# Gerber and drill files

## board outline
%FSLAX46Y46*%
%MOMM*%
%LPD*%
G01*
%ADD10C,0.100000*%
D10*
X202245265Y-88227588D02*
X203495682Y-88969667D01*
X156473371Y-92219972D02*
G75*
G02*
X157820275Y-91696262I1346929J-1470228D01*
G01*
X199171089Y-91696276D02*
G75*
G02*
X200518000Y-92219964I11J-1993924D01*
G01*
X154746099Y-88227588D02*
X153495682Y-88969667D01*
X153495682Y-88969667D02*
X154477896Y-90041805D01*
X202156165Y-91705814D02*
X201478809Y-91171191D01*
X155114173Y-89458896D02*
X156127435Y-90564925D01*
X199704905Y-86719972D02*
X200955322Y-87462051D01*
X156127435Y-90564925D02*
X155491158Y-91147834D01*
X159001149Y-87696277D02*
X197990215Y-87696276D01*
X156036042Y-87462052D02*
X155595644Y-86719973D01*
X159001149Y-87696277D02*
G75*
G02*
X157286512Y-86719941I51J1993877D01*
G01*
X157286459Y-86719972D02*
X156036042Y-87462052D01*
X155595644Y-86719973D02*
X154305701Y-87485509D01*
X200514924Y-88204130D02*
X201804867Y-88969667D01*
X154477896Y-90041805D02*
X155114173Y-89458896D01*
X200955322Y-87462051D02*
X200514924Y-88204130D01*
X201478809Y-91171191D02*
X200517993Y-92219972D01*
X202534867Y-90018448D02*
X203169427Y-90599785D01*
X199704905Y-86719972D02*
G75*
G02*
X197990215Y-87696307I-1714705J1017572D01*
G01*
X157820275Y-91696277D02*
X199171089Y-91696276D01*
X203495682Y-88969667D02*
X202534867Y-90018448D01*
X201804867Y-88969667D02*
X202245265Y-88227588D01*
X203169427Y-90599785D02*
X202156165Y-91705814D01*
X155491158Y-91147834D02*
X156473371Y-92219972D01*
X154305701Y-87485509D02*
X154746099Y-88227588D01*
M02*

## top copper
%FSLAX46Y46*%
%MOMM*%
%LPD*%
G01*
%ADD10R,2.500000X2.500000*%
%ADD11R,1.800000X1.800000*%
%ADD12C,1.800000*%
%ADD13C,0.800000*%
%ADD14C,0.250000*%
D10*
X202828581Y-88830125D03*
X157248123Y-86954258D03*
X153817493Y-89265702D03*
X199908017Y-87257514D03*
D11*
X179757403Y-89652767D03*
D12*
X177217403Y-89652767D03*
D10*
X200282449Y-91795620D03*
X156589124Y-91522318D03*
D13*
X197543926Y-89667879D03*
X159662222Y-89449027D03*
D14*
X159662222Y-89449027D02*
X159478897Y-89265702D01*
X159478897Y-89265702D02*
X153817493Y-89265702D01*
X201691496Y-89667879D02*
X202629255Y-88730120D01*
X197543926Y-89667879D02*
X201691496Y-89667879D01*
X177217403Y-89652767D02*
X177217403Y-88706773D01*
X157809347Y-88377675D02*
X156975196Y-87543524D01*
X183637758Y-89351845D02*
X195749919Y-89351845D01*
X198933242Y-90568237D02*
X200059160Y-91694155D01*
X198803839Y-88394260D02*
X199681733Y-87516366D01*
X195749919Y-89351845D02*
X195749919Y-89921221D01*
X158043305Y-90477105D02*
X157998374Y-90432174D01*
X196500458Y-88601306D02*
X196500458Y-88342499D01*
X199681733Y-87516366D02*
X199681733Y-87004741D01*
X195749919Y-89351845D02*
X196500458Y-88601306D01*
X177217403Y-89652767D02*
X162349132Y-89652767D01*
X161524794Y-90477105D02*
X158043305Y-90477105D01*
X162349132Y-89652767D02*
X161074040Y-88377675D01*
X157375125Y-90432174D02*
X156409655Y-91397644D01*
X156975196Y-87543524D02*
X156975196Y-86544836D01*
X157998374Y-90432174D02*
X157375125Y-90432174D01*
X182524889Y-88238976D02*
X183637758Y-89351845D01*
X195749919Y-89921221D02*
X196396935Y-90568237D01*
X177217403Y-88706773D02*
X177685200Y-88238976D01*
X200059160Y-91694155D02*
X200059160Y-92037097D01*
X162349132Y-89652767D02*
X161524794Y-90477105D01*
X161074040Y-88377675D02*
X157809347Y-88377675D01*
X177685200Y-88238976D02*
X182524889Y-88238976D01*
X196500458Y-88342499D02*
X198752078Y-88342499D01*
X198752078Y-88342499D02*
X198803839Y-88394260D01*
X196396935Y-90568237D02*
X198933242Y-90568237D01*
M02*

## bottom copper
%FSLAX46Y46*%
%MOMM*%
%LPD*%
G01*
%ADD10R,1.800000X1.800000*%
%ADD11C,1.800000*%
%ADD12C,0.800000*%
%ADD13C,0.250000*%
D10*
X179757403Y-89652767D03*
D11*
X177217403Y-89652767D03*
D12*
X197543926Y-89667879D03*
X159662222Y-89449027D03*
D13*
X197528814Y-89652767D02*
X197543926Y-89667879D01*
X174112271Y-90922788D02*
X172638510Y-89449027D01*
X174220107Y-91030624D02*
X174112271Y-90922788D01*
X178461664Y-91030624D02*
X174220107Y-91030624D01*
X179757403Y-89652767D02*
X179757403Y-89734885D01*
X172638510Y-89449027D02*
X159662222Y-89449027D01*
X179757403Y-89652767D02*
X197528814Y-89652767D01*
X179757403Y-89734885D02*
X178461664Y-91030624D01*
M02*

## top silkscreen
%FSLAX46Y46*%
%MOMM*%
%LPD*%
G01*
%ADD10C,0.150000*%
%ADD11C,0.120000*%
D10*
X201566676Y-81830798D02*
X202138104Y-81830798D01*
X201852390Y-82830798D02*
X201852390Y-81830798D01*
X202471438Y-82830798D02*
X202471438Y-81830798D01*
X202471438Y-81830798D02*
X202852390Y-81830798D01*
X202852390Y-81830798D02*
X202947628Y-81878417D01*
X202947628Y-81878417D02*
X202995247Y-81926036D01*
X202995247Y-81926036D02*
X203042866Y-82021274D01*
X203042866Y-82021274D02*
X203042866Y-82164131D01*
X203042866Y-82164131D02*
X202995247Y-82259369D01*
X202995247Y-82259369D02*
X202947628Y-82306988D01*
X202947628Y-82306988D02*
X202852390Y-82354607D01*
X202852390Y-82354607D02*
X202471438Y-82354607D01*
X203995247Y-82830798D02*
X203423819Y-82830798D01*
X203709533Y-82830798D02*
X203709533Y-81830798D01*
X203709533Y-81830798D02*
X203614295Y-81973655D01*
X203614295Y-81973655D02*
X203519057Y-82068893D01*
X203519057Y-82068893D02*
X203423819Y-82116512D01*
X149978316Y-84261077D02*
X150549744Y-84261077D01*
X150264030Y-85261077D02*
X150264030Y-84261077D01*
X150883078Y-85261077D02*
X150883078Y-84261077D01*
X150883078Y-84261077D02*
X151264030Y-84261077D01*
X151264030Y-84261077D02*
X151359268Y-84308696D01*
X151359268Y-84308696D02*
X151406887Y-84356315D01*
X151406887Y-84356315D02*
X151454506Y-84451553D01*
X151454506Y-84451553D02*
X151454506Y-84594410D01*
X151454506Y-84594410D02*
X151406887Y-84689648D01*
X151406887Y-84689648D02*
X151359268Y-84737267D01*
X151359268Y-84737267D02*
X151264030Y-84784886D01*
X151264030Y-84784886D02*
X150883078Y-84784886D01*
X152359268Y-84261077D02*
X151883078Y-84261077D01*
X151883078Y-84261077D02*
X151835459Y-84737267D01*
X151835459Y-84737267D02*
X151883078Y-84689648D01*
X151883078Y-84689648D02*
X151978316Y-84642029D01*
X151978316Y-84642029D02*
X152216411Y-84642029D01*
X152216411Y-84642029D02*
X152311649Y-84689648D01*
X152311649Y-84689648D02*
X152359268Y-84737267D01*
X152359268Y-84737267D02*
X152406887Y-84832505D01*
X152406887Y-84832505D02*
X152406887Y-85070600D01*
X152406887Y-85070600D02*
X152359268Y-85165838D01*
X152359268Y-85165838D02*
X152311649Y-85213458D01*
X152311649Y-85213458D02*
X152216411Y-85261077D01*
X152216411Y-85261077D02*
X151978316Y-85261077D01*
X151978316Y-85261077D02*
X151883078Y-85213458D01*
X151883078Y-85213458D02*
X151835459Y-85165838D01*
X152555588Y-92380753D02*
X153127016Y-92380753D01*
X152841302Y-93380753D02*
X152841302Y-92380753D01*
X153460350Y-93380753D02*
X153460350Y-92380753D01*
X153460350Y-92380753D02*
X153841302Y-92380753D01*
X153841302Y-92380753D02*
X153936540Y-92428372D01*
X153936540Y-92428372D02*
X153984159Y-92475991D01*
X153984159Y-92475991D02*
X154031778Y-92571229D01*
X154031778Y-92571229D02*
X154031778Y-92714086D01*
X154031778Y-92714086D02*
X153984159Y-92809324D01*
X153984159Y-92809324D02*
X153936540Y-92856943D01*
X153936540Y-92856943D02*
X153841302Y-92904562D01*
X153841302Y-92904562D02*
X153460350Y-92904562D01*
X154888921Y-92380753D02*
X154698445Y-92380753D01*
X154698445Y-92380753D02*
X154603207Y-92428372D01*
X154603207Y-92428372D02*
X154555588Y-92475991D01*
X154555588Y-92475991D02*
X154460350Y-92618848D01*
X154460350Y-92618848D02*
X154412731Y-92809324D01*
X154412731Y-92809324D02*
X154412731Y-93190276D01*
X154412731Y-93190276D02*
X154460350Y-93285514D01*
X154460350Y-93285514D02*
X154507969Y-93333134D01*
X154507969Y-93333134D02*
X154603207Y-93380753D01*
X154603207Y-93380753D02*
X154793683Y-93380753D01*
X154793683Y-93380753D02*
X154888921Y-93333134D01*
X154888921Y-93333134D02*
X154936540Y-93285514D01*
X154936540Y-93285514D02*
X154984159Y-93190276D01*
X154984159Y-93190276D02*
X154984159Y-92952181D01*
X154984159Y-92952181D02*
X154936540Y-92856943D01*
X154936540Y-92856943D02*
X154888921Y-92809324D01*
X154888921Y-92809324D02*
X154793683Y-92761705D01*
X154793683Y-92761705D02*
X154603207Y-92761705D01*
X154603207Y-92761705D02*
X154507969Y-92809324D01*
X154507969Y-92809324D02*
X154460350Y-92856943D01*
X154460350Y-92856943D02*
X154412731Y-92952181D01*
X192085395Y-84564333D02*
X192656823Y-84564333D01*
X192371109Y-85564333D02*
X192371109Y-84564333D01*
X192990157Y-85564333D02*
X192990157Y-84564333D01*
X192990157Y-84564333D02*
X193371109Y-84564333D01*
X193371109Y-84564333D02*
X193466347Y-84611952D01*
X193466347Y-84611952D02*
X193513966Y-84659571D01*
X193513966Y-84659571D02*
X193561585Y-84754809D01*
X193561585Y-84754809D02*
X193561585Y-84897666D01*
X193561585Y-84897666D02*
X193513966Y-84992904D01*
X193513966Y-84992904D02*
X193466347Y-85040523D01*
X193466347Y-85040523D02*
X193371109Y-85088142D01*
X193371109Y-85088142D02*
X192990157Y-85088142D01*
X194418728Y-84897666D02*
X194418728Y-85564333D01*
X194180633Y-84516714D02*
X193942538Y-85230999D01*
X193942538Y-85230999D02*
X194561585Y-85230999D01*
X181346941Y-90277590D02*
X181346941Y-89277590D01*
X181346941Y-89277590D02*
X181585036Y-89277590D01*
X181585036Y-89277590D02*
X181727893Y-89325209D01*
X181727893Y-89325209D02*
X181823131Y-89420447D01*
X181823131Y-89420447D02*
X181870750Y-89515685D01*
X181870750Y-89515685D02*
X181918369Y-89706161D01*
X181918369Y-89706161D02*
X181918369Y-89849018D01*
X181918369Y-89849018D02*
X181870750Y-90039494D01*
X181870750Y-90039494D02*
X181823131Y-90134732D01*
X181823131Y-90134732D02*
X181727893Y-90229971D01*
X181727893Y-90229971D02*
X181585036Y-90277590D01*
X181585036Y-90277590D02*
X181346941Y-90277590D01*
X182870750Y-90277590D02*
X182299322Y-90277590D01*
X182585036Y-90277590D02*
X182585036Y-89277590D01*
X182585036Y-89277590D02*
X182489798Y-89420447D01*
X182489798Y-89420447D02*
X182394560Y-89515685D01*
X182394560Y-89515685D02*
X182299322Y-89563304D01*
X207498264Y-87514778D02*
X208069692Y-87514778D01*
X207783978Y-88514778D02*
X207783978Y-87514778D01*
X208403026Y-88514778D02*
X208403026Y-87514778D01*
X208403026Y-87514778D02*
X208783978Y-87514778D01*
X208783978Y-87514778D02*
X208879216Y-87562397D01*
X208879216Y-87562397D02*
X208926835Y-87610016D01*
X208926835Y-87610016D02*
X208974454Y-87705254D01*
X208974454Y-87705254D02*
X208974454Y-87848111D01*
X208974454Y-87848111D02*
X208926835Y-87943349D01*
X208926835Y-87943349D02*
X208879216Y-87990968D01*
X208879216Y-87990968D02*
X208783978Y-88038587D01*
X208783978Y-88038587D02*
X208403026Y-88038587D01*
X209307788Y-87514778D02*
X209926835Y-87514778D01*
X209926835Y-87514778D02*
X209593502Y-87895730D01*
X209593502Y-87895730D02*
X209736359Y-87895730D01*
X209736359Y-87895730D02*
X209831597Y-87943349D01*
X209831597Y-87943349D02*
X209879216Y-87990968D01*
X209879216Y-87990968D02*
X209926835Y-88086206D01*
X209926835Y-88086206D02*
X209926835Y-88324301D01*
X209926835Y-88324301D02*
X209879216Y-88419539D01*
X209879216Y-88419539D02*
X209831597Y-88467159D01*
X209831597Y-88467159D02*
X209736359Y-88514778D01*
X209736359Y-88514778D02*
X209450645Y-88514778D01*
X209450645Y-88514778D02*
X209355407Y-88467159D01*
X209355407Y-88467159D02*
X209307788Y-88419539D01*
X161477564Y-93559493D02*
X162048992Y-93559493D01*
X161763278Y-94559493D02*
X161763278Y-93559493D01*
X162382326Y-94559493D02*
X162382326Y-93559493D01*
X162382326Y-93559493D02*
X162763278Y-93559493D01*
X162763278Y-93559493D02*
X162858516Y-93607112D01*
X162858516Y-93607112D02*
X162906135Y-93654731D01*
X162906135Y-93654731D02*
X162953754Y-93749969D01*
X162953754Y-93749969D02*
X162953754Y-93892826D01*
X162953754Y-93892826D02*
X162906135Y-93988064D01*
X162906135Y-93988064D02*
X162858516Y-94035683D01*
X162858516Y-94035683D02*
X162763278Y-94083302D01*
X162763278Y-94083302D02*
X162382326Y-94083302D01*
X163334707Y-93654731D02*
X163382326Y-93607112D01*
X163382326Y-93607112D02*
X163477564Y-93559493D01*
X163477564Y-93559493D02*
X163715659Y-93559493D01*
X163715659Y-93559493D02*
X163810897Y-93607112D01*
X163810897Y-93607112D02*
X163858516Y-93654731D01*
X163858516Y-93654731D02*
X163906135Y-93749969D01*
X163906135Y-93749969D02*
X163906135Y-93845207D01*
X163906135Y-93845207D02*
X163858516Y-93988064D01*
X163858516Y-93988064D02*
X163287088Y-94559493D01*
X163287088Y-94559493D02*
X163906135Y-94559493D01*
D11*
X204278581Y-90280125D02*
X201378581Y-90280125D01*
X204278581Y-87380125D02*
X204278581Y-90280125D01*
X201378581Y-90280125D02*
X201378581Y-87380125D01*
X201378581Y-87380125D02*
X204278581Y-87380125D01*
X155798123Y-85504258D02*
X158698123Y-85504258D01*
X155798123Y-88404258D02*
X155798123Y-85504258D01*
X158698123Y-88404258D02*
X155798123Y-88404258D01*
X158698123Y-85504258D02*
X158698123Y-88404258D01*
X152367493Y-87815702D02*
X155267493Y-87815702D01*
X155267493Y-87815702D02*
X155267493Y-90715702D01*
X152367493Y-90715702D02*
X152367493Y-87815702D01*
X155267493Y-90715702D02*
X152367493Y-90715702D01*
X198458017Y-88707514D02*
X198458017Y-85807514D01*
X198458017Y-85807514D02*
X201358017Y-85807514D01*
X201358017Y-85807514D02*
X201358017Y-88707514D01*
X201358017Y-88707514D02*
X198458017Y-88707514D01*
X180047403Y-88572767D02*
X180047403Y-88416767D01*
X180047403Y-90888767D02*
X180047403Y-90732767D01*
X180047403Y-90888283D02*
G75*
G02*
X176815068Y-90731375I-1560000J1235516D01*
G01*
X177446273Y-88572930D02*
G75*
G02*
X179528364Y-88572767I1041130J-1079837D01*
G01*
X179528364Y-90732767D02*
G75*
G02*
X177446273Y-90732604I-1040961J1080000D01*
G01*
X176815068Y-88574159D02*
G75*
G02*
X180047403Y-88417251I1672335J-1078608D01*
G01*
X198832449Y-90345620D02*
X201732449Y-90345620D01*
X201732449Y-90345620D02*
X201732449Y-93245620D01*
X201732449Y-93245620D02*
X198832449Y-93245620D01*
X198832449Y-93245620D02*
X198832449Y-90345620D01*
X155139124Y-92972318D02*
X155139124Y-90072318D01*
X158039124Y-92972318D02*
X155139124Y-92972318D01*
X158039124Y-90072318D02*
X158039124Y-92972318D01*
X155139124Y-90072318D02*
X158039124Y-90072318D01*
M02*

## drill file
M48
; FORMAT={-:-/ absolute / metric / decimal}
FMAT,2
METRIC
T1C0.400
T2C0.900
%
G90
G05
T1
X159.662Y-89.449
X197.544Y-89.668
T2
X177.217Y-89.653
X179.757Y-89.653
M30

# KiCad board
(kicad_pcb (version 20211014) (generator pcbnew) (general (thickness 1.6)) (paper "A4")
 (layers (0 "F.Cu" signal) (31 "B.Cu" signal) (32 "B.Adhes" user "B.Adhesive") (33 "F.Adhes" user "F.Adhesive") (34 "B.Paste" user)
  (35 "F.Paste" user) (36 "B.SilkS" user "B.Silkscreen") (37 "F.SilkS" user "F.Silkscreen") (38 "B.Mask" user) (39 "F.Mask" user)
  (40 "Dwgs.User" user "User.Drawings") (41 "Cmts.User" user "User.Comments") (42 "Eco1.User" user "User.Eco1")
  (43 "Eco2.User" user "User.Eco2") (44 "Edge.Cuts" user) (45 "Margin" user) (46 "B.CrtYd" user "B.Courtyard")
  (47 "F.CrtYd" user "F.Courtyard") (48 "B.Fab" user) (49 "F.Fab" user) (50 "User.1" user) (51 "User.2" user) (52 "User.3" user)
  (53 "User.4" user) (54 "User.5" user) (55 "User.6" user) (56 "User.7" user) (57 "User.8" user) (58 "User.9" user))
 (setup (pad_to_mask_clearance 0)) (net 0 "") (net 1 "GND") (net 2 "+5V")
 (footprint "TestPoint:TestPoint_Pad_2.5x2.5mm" (layer "F.Cu") (at 202.828581 88.830125)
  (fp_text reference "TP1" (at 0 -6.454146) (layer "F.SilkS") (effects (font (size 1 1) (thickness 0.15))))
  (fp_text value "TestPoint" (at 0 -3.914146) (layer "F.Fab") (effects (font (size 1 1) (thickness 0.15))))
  (fp_line (start 1.45 1.45) (end -1.45 1.45) (layer "F.SilkS") (width 0.12))
  (fp_line (start 1.45 -1.45) (end 1.45 1.45) (layer "F.SilkS") (width 0.12))
  (fp_line (start -1.45 1.45) (end -1.45 -1.45) (layer "F.SilkS") (width 0.12))
  (fp_line (start -1.45 -1.45) (end 1.45 -1.45) (layer "F.SilkS") (width 0.12))
  (pad "1" smd rect (at 0 0) (size 2.5 2.5) (layers "F.Cu" "F.Mask") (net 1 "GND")))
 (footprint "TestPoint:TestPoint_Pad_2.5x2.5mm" (layer "F.Cu") (at 157.248123 86.954258)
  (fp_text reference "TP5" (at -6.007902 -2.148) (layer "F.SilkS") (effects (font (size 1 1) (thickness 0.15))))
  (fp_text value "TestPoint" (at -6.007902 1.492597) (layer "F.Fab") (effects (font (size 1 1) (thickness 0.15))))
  (fp_line (start -1.45 -1.45) (end 1.45 -1.45) (layer "F.SilkS") (width 0.12))
  (fp_line (start -1.45 1.45) (end -1.45 -1.45) (layer "F.SilkS") (width 0.12))
  (fp_line (start 1.45 1.45) (end -1.45 1.45) (layer "F.SilkS") (width 0.12))
  (fp_line (start 1.45 -1.45) (end 1.45 1.45) (layer "F.SilkS") (width 0.12))
  (pad "1" smd rect (at 0 0) (size 2.5 2.5) (layers "F.Cu" "F.Mask") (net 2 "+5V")))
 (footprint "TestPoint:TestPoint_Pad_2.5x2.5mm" (layer "F.Cu") (at 153.817493 89.265702)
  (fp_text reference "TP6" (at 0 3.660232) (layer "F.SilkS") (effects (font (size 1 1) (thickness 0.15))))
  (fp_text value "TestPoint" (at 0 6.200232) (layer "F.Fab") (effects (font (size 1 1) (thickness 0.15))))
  (fp_line (start -1.45 -1.45) (end 1.45 -1.45) (layer "F.SilkS") (width 0.12))
  (fp_line (start 1.45 -1.45) (end 1.45 1.45) (layer "F.SilkS") (width 0.12))
  (fp_line (start -1.45 1.45) (end -1.45 -1.45) (layer "F.SilkS") (width 0.12))
  (fp_line (start 1.45 1.45) (end -1.45 1.45) (layer "F.SilkS") (width 0.12))
  (pad "1" smd rect (at 0 0) (size 2.5 2.5) (layers "F.Cu" "F.Mask") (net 1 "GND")))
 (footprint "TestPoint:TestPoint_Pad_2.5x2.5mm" (layer "F.Cu") (at 199.908017 87.257514)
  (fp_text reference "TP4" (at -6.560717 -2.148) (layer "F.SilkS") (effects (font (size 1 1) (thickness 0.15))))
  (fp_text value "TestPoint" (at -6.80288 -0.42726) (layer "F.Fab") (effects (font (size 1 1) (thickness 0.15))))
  (fp_line (start -1.45 1.45) (end -1.45 -1.45) (layer "F.SilkS") (width 0.12))
  (fp_line (start -1.45 -1.45) (end 1.45 -1.45) (layer "F.SilkS") (width 0.12))
  (fp_line (start 1.45 -1.45) (end 1.45 1.45) (layer "F.SilkS") (width 0.12))
  (fp_line (start 1.45 1.45) (end -1.45 1.45) (layer "F.SilkS") (width 0.12))
  (pad "1" smd rect (at 0 0) (size 2.5 2.5) (layers "F.Cu" "F.Mask") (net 2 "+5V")))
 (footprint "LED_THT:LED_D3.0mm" (layer "F.Cu") (at 179.757403 89.652767 180)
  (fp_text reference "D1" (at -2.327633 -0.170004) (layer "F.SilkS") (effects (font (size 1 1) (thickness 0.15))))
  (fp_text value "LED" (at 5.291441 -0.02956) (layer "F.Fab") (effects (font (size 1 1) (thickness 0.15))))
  (fp_line (start -0.29 1.08) (end -0.29 1.236) (layer "F.SilkS") (width 0.12))
  (fp_line (start -0.29 -1.236) (end -0.29 -1.08) (layer "F.SilkS") (width 0.12))
  (fp_arc (start -0.29 -1.235516) (mid 1.366487 -1.987659) (end 2.942335 -1.078608) (layer "F.SilkS") (width 0.12))
  (fp_arc (start 2.31113 1.079837) (mid 1.270117 1.5) (end 0.229039 1.08) (layer "F.SilkS") (width 0.12))
  (fp_arc (start 0.229039 -1.08) (mid 1.270117 -1.5) (end 2.31113 -1.079837) (layer "F.SilkS") (width 0.12))
  (fp_arc (start 2.942335 1.078608) (mid 1.366487 1.987659) (end -0.29 1.235516) (layer "F.SilkS") (width 0.12))
  (pad "1" thru_hole rect (at 0 0 180) (size 1.8 1.8) (drill 0.9) (layers *.Cu *.Mask) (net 1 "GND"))
  (pad "2" thru_hole circle (at 2.54 0 180) (size 1.8 1.8) (drill 0.9) (layers *.Cu *.Mask) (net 2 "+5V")))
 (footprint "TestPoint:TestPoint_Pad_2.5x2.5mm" (layer "F.Cu") (at 200.282449 91.79562)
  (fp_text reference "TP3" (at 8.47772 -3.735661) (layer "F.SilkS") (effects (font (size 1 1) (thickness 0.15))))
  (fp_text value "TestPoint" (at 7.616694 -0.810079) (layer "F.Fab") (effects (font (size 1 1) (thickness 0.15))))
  (fp_line (start -1.45 -1.45) (end 1.45 -1.45) (layer "F.SilkS") (width 0.12))
  (fp_line (start 1.45 -1.45) (end 1.45 1.45) (layer "F.SilkS") (width 0.12))
  (fp_line (start 1.45 1.45) (end -1.45 1.45) (layer "F.SilkS") (width 0.12))
  (fp_line (start -1.45 1.45) (end -1.45 -1.45) (layer "F.SilkS") (width 0.12))
  (pad "1" smd rect (at 0 0) (size 2.5 2.5) (layers "F.Cu" "F.Mask") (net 2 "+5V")))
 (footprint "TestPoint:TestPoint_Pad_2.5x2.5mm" (layer "F.Cu") (at 156.589124 91.522318)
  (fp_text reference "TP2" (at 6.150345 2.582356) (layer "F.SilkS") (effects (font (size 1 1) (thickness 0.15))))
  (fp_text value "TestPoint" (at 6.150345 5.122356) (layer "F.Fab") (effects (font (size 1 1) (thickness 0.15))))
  (fp_line (start -1.45 1.45) (end -1.45 -1.45) (layer "F.SilkS") (width 0.12))
  (fp_line (start 1.45 1.45) (end -1.45 1.45) (layer "F.SilkS") (width 0.12))
  (fp_line (start 1.45 -1.45) (end 1.45 1.45) (layer "F.SilkS") (width 0.12))
  (fp_line (start -1.45 -1.45) (end 1.45 -1.45) (layer "F.SilkS") (width 0.12))
  (pad "1" smd rect (at 0 0) (size 2.5 2.5) (layers "F.Cu" "F.Mask") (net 2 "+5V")))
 (gr_line (start 202.245265 88.227588) (end 203.495682 88.969667) (layer "Edge.Cuts") (width 0.1))
 (gr_arc (start 156.473371 92.219972) (mid 157.097709 91.831807) (end 157.820275 91.696277) (layer "Edge.Cuts") (width 0.1))
 (gr_arc (start 199.171089 91.696276) (mid 199.893655 91.831806) (end 200.517993 92.219972) (layer "Edge.Cuts") (width 0.1))
 (gr_line (start 154.746099 88.227588) (end 153.495682 88.969667) (layer "Edge.Cuts") (width 0.1))
 (gr_line (start 153.495682 88.969667) (end 154.477896 90.041805) (layer "Edge.Cuts") (width 0.1))
 (gr_line (start 202.156165 91.705814) (end 201.478809 91.171191) (layer "Edge.Cuts") (width 0.1))
 (gr_line (start 155.114173 89.458896) (end 156.127435 90.564925) (layer "Edge.Cuts") (width 0.1))
 (gr_line (start 199.704905 86.719972) (end 200.955322 87.462051) (layer "Edge.Cuts") (width 0.1))
 (gr_line (start 156.127435 90.564925) (end 155.491158 91.147834) (layer "Edge.Cuts") (width 0.1))
 (gr_line (start 159.001149 87.696277) (end 197.990215 87.696276) (layer "Edge.Cuts") (width 0.1))
 (gr_line (start 156.036042 87.462052) (end 155.595644 86.719973) (layer "Edge.Cuts") (width 0.1))
 (gr_arc (start 159.001149 87.696277) (mid 158.014573 87.435094) (end 157.286459 86.719972) (layer "Edge.Cuts") (width 0.1))
 (gr_line (start 157.286459 86.719972) (end 156.036042 87.462052) (layer "Edge.Cuts") (width 0.1))
 (gr_line (start 155.595644 86.719973) (end 154.305701 87.485509) (layer "Edge.Cuts") (width 0.1))
 (gr_line (start 200.514924 88.20413) (end 201.804867 88.969667) (layer "Edge.Cuts") (width 0.1))
 (gr_line (start 154.477896 90.041805) (end 155.114173 89.458896) (layer "Edge.Cuts") (width 0.1))
 (gr_line (start 200.955322 87.462051) (end 200.514924 88.20413) (layer "Edge.Cuts") (width 0.1))
 (gr_line (start 201.478809 91.171191) (end 200.517993 92.219972) (layer "Edge.Cuts") (width 0.1))
 (gr_line (start 202.534867 90.018448) (end 203.169427 90.599785) (layer "Edge.Cuts") (width 0.1))
 (gr_arc (start 199.704905 86.719972) (mid 198.976791 87.435094) (end 197.990215 87.696276) (layer "Edge.Cuts") (width 0.1))
 (gr_line (start 157.820275 91.696277) (end 199.171089 91.696276) (layer "Edge.Cuts") (width 0.1))
 (gr_line (start 203.495682 88.969667) (end 202.534867 90.018448) (layer "Edge.Cuts") (width 0.1))
 (gr_line (start 201.804867 88.969667) (end 202.245265 88.227588) (layer "Edge.Cuts") (width 0.1))
 (gr_line (start 203.169427 90.599785) (end 202.156165 91.705814) (layer "Edge.Cuts") (width 0.1))
 (gr_line (start 155.491158 91.147834) (end 156.473371 92.219972) (layer "Edge.Cuts") (width 0.1))
 (gr_line (start 154.305701 87.485509) (end 154.746099 88.227588) (layer "Edge.Cuts") (width 0.1))
 (segment (start 159.662222 89.449027) (end 159.478897 89.265702) (width 0.25) (layer "F.Cu") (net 1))
 (segment (start 159.478897 89.265702) (end 153.817493 89.265702) (width 0.25) (layer "F.Cu") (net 1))
 (segment (start 201.691496 89.667879) (end 202.629255 88.73012) (width 0.25) (layer "F.Cu") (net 1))
 (segment (start 197.543926 89.667879) (end 201.691496 89.667879) (width 0.25) (layer "F.Cu") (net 1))
 (via (at 197.543926 89.667879) (size 0.8) (drill 0.4) (layers "F.Cu" "B.Cu") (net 1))
 (via (at 159.662222 89.449027) (size 0.8) (drill 0.4) (layers "F.Cu" "B.Cu") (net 1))
 (segment (start 197.528814 89.652767) (end 197.543926 89.667879) (width 0.25) (layer "B.Cu") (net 1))
 (segment (start 174.112271 90.922788) (end 172.63851 89.449027) (width 0.25) (layer "B.Cu") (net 1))
 (segment (start 174.220107 91.030624) (end 174.112271 90.922788) (width 0.25) (layer "B.Cu") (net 1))
 (segment (start 178.461664 91.030624) (end 174.220107 91.030624) (width 0.25) (layer "B.Cu") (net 1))
 (segment (start 179.757403 89.652767) (end 179.757403 89.734885) (width 0.25) (layer "B.Cu") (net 1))
 (segment (start 172.63851 89.449027) (end 159.662222 89.449027) (width 0.25) (layer "B.Cu") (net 1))
 (segment (start 179.757403 89.652767) (end 197.528814 89.652767) (width 0.25) (layer "B.Cu") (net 1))
 (segment (start 179.757403 89.734885) (end 178.461664 91.030624) (width 0.25) (layer "B.Cu") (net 1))
 (segment (start 177.217403 89.652767) (end 177.217403 88.706773) (width 0.25) (layer "F.Cu") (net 2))
 (segment (start 157.809347 88.377675) (end 156.975196 87.543524) (width 0.25) (layer "F.Cu") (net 2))
 (segment (start 183.637758 89.351845) (end 195.749919 89.351845) (width 0.25) (layer "F.Cu") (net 2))
 (segment (start 198.933242 90.568237) (end 200.05916 91.694155) (width 0.25) (layer "F.Cu") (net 2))
 (segment (start 198.803839 88.39426) (end 199.681733 87.516366) (width 0.25) (layer "F.Cu") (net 2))
 (segment (start 195.749919 89.351845) (end 195.749919 89.921221) (width 0.25) (layer "F.Cu") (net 2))
 (segment (start 158.043305 90.477105) (end 157.998374 90.432174) (width 0.25) (layer "F.Cu") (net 2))
 (segment (start 196.500458 88.601306) (end 196.500458 88.342499) (width 0.25) (layer "F.Cu") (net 2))
 (segment (start 199.681733 87.516366) (end 199.681733 87.004741) (width 0.25) (layer "F.Cu") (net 2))
 (segment (start 195.749919 89.351845) (end 196.500458 88.601306) (width 0.25) (layer "F.Cu") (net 2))
 (segment (start 177.217403 89.652767) (end 162.349132 89.652767) (width 0.25) (layer "F.Cu") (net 2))
 (segment (start 161.524794 90.477105) (end 158.043305 90.477105) (width 0.25) (layer "F.Cu") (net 2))
 (segment (start 162.349132 89.652767) (end 161.07404 88.377675) (width 0.25) (layer "F.Cu") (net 2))
 (segment (start 157.375125 90.432174) (end 156.409655 91.397644) (width 0.25) (layer "F.Cu") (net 2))
 (segment (start 156.975196 87.543524) (end 156.975196 86.544836) (width 0.25) (layer "F.Cu") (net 2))
 (segment (start 157.998374 90.432174) (end 157.375125 90.432174) (width 0.25) (layer "F.Cu") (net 2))
 (segment (start 182.524889 88.238976) (end 183.637758 89.351845) (width 0.25) (layer "F.Cu") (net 2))
 (segment (start 195.749919 89.921221) (end 196.396935 90.568237) (width 0.25) (layer "F.Cu") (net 2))
 (segment (start 177.217403 88.706773) (end 177.6852 88.238976) (width 0.25) (layer "F.Cu") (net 2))
 (segment (start 200.05916 91.694155) (end 200.05916 92.037097) (width 0.25) (layer "F.Cu") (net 2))
 (segment (start 162.349132 89.652767) (end 161.524794 90.477105) (width 0.25) (layer "F.Cu") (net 2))
 (segment (start 161.07404 88.377675) (end 157.809347 88.377675) (width 0.25) (layer "F.Cu") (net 2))
 (segment (start 177.6852 88.238976) (end 182.524889 88.238976) (width 0.25) (layer "F.Cu") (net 2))
 (segment (start 196.500458 88.342499) (end 198.752078 88.342499) (width 0.25) (layer "F.Cu") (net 2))
 (segment (start 198.752078 88.342499) (end 198.803839 88.39426) (width 0.25) (layer "F.Cu") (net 2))
 (segment (start 196.396935 90.568237) (end 198.933242 90.568237) (width 0.25) (layer "F.Cu") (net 2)))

